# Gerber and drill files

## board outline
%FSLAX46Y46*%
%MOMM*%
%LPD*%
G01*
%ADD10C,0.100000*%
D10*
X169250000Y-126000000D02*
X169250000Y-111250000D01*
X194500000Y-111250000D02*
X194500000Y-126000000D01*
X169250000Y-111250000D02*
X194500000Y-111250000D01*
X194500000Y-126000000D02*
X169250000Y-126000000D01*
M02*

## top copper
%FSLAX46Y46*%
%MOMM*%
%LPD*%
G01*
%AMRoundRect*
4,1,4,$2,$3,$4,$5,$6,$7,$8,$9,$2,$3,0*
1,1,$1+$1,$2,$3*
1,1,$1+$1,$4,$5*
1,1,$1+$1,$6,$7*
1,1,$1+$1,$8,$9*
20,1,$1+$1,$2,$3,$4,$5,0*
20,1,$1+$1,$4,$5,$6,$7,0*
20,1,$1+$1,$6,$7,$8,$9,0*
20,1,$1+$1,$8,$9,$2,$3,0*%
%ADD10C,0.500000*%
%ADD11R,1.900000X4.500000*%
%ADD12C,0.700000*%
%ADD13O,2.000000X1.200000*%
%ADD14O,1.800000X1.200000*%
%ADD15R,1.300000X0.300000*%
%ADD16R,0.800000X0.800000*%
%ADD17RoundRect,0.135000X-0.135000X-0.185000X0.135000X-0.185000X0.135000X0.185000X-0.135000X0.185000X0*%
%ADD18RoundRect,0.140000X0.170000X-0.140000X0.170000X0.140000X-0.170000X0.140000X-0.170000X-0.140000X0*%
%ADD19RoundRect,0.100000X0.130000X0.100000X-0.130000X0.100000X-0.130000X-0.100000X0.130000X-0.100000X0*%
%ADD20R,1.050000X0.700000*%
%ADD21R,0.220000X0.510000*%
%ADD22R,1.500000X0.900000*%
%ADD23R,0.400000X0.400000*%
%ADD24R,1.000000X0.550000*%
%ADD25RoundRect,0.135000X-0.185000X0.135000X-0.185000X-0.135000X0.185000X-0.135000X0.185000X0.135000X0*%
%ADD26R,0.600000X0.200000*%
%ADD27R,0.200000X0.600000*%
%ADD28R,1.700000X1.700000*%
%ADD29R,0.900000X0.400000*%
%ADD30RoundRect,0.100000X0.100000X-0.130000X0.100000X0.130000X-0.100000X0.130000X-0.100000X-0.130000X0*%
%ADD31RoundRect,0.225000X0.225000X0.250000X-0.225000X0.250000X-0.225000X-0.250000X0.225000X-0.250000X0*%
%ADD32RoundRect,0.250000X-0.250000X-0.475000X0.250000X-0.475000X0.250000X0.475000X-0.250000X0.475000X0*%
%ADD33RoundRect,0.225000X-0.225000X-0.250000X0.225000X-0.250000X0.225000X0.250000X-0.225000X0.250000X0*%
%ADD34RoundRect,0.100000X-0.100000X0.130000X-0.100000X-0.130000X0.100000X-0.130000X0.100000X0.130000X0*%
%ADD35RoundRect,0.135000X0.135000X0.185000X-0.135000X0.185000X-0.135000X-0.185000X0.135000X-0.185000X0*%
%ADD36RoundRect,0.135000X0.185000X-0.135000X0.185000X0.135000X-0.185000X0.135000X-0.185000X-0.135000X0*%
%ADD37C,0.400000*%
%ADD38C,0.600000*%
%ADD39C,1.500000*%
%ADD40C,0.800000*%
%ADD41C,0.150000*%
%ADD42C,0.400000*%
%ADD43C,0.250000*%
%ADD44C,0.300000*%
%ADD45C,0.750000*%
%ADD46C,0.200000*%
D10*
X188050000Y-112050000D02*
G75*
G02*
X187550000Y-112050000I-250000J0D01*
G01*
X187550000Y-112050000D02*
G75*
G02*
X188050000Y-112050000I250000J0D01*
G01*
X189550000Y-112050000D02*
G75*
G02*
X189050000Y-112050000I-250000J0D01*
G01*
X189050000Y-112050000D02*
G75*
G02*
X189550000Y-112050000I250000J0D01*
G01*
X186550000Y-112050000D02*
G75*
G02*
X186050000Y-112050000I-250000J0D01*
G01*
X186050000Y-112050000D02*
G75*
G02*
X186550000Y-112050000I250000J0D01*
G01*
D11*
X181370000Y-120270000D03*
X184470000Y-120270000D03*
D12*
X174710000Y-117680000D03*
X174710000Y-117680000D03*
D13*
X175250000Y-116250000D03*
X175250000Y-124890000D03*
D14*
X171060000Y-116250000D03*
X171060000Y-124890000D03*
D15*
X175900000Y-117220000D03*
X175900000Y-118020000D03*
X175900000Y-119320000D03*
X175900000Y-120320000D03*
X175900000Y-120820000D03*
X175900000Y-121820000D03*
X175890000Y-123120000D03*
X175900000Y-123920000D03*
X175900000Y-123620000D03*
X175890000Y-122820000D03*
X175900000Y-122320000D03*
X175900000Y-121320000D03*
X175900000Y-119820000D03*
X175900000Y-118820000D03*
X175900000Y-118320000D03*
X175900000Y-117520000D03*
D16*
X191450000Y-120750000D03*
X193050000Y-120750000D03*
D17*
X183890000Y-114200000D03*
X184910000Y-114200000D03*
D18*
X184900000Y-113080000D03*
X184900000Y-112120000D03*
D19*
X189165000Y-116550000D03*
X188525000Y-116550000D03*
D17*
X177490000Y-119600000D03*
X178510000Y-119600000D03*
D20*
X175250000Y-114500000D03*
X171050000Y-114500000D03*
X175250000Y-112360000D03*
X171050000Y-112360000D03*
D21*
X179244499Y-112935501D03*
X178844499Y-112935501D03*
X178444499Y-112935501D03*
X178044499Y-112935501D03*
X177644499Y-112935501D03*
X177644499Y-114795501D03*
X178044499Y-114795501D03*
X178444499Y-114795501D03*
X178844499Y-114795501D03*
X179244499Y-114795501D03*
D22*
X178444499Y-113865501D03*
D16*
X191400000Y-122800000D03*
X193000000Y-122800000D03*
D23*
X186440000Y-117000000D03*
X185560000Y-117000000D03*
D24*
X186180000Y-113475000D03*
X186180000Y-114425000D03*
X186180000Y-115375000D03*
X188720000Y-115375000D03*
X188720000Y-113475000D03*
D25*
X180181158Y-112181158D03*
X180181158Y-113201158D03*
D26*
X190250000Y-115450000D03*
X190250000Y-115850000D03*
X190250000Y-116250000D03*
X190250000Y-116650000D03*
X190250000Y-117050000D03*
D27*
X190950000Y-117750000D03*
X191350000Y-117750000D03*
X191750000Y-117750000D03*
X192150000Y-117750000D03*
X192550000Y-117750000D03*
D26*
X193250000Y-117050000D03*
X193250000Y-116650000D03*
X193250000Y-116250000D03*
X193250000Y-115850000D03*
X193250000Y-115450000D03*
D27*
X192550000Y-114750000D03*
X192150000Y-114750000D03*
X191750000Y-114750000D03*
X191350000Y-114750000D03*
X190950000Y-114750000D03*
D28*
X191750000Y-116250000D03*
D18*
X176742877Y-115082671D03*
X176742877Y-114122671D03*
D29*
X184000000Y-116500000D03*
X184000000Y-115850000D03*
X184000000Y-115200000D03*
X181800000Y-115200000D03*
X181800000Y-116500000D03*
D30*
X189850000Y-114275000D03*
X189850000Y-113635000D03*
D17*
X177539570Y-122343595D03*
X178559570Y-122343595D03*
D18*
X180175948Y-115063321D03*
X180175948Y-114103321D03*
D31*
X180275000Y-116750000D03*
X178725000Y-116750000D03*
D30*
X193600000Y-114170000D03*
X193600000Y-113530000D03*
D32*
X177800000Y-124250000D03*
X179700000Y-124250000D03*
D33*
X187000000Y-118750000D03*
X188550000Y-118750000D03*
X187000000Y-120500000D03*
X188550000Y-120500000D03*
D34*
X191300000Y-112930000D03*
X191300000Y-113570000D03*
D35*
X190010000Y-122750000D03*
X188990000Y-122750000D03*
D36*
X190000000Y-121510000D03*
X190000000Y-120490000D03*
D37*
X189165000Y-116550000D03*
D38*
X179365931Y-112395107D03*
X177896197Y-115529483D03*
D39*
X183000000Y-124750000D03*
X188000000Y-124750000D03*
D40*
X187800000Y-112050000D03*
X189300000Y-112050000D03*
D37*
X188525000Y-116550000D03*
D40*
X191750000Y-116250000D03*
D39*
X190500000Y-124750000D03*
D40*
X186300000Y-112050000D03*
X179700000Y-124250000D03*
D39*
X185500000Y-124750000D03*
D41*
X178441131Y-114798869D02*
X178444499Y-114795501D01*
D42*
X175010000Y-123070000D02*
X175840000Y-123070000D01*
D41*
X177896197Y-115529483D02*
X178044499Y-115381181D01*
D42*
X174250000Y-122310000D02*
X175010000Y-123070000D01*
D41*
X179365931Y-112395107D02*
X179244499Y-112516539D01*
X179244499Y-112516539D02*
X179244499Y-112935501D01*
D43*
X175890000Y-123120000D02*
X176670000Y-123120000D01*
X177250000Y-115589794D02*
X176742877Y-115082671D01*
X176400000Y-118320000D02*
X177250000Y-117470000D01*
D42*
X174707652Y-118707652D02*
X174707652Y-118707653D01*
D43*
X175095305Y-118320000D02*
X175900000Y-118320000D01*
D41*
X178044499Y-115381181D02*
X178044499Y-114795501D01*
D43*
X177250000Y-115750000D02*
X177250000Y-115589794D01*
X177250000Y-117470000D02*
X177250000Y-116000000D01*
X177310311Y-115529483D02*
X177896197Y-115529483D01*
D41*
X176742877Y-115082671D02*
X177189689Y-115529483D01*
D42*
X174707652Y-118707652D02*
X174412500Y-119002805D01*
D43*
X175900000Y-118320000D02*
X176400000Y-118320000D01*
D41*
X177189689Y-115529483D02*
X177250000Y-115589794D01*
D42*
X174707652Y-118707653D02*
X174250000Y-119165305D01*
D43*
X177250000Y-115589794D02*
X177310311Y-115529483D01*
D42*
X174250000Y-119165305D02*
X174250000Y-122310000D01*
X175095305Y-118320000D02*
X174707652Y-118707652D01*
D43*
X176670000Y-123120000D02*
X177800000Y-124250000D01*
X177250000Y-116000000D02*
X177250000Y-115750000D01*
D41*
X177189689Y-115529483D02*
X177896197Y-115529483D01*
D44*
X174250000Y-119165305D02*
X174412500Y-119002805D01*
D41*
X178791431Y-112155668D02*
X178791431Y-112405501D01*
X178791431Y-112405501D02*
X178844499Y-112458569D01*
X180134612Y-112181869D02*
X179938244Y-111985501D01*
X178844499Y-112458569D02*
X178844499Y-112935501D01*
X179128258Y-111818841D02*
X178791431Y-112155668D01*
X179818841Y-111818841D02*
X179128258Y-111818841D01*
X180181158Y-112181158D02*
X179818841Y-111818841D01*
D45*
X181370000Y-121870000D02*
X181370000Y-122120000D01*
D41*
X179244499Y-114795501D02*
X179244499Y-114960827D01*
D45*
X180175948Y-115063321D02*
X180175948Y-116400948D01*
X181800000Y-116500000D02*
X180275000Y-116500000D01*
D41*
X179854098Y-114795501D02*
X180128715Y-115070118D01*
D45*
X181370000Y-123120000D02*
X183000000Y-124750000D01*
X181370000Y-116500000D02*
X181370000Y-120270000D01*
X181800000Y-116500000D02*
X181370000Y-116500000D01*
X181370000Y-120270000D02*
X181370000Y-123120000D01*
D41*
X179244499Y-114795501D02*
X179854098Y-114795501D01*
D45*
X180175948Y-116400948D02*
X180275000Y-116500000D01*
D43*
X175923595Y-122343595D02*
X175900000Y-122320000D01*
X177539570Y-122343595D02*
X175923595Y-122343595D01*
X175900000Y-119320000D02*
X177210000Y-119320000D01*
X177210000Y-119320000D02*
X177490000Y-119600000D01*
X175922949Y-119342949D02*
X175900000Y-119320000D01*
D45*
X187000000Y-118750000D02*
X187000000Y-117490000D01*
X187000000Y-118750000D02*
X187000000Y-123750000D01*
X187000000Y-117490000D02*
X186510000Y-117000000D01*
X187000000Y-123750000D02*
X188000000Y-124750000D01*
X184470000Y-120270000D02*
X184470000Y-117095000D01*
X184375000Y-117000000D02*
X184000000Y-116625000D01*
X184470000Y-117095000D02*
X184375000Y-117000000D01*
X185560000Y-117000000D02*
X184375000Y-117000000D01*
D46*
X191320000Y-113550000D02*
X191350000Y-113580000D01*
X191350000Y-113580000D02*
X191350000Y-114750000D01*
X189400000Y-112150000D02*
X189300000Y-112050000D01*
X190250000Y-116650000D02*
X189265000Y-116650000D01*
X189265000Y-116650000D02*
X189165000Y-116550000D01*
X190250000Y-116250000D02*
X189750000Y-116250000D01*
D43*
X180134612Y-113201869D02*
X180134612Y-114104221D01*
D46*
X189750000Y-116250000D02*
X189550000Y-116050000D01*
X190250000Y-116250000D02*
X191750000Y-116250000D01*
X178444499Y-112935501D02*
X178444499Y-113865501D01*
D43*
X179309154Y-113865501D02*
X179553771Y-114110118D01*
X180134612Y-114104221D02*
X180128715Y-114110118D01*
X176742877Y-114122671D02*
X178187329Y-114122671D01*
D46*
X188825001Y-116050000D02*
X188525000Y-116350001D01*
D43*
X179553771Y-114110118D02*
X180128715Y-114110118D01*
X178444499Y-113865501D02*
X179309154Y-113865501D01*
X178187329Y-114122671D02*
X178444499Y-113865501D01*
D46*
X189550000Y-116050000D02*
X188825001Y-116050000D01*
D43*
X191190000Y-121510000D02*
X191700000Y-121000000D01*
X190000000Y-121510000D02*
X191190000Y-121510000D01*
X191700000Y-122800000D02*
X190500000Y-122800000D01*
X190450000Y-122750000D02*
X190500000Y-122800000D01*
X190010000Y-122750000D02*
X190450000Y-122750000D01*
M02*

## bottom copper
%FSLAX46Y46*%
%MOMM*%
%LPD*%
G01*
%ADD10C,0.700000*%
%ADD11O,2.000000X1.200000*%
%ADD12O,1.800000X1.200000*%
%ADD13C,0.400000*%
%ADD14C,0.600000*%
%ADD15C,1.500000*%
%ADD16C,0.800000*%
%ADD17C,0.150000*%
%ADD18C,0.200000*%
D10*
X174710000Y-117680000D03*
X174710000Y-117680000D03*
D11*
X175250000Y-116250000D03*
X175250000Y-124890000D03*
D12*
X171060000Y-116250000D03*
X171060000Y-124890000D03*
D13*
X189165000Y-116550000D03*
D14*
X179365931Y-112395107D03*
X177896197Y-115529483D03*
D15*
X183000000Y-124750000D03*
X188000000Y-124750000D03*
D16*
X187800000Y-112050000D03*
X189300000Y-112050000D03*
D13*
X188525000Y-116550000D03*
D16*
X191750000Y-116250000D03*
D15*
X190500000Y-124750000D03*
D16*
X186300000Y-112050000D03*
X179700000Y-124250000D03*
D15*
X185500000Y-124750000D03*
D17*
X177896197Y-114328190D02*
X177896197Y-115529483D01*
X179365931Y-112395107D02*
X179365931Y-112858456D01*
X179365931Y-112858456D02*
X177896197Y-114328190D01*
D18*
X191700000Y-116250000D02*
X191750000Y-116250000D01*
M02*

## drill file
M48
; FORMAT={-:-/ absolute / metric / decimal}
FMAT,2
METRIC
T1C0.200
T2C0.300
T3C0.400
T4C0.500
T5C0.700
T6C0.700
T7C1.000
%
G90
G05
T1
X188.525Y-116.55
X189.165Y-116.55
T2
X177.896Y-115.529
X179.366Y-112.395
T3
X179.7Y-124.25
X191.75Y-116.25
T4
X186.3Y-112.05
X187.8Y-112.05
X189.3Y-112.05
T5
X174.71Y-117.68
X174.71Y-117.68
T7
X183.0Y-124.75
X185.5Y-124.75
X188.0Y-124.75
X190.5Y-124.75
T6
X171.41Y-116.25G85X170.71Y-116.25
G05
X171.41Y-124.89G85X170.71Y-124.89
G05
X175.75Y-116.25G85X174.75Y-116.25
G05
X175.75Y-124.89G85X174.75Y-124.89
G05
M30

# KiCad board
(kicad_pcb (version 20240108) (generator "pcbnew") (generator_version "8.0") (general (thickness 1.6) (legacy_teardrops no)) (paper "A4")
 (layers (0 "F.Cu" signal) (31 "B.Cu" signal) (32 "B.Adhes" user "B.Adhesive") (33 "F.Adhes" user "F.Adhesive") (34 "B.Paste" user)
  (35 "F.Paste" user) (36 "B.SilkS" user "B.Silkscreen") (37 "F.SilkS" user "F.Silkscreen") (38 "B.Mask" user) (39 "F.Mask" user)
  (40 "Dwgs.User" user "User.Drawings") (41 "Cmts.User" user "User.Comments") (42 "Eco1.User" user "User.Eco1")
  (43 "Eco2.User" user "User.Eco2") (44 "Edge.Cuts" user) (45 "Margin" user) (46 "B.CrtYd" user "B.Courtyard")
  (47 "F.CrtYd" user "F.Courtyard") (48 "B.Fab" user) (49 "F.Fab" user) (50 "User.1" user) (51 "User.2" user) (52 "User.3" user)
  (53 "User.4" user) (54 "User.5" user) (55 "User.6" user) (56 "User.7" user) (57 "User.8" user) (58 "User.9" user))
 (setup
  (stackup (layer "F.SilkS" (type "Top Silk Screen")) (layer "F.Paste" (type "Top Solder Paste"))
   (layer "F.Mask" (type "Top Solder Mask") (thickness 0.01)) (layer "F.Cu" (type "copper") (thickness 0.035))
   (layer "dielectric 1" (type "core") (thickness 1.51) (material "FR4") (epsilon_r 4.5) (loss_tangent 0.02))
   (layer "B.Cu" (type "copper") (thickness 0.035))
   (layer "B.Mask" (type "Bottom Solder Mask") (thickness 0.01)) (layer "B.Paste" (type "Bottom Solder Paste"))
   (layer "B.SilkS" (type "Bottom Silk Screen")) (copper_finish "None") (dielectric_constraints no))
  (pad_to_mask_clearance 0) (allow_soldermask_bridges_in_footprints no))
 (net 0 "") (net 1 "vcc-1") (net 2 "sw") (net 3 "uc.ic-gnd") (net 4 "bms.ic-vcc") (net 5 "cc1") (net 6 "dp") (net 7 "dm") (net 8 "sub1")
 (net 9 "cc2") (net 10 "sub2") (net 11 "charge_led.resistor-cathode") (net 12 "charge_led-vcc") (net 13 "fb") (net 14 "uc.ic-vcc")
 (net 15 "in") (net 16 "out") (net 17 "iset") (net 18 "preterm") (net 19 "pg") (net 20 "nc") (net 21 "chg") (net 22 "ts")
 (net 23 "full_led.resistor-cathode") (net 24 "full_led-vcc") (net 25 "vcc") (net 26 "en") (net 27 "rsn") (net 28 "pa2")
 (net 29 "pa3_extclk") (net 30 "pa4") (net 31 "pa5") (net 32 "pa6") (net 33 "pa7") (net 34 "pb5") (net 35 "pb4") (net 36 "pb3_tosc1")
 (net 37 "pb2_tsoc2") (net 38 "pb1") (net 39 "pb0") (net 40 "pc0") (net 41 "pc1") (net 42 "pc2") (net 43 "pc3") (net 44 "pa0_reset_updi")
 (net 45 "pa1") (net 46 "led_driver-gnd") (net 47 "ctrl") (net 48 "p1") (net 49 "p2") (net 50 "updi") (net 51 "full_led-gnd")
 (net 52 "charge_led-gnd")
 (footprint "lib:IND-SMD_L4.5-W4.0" (layer "F.Cu") (at 182.92 120.27)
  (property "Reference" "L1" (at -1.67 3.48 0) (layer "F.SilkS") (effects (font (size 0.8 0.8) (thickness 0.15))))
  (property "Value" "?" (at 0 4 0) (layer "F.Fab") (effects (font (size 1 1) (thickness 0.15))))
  (pad "1" smd rect (at -1.55 0) (size 1.9 4.5) (layers "F.Cu" "F.Paste" "F.Mask") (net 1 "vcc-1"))
  (pad "2" smd rect (at 1.55 0) (size 1.9 4.5) (layers "F.Cu" "F.Paste" "F.Mask") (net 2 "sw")))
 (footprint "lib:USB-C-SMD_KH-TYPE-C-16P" (layer "F.Cu") (at 173.48 120.57 -90)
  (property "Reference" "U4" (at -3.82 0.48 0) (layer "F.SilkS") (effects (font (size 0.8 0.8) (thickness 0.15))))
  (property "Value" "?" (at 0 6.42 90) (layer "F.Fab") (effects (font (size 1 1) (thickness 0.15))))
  (pad "" thru_hole circle (at -2.89 -1.23 270) (size 0.7 0.7) (drill 0.7) (layers "*.Cu" "*.Mask") (remove_unused_layers no))
  (pad "" thru_hole circle (at -2.89 -1.23 270) (size 0.7 0.7) (drill 0.7) (layers "*.Cu" "*.Mask") (remove_unused_layers no))
  (pad "1" thru_hole oval (at -4.32 -1.77 270) (size 1.2 2) (drill oval 0.700024 1.699997) (layers "*.Cu" "*.Mask")
   (remove_unused_layers no) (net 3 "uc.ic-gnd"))
  (pad "2" thru_hole oval (at 4.32 -1.77 270) (size 1.2 2) (drill oval 0.700024 1.699997) (layers "*.Cu" "*.Mask") (remove_unused_layers no)
   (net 3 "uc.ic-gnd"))
  (pad "3" thru_hole oval (at -4.32 2.42 270) (size 1.2 1.8) (drill oval 0.700024 1.399997) (layers "*.Cu" "*.Mask")
   (remove_unused_layers no) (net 3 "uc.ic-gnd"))
  (pad "4" thru_hole oval (at 4.32 2.42 270) (size 1.2 1.8) (drill oval 0.700024 1.399997) (layers "*.Cu" "*.Mask")
   (remove_unused_layers no) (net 3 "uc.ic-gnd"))
  (pad "A1" smd rect (at -3.35 -2.42 270) (size 0.3 1.3) (layers "F.Cu" "F.Paste" "F.Mask") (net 3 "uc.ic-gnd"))
  (pad "A4" smd rect (at -2.55 -2.42 270) (size 0.3 1.3) (layers "F.Cu" "F.Paste" "F.Mask") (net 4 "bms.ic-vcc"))
  (pad "A5" smd rect (at -1.25 -2.42 270) (size 0.3 1.3) (layers "F.Cu" "F.Paste" "F.Mask") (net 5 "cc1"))
  (pad "A6" smd rect (at -0.25 -2.42 270) (size 0.3 1.3) (layers "F.Cu" "F.Paste" "F.Mask") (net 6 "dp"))
  (pad "A7" smd rect (at 0.25 -2.42 270) (size 0.3 1.3) (layers "F.Cu" "F.Paste" "F.Mask") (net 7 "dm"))
  (pad "A8" smd rect (at 1.25 -2.42 270) (size 0.3 1.3) (layers "F.Cu" "F.Paste" "F.Mask") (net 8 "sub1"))
  (pad "A9" smd rect (at 2.55 -2.41 270) (size 0.3 1.3) (layers "F.Cu" "F.Paste" "F.Mask") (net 4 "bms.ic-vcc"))
  (pad "A12" smd rect (at 3.35 -2.42 270) (size 0.3 1.3) (layers "F.Cu" "F.Paste" "F.Mask") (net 3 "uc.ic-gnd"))
  (pad "B1" smd rect (at 3.05 -2.42 270) (size 0.3 1.3) (layers "F.Cu" "F.Paste" "F.Mask") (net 3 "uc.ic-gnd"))
  (pad "B4" smd rect (at 2.25 -2.41 270) (size 0.3 1.3) (layers "F.Cu" "F.Paste" "F.Mask") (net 4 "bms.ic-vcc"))
  (pad "B5" smd rect (at 1.75 -2.42 270) (size 0.3 1.3) (layers "F.Cu" "F.Paste" "F.Mask") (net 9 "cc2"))
  (pad "B6" smd rect (at 0.75 -2.42 270) (size 0.3 1.3) (layers "F.Cu" "F.Paste" "F.Mask") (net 6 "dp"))
  (pad "B7" smd rect (at -0.75 -2.42 270) (size 0.3 1.3) (layers "F.Cu" "F.Paste" "F.Mask") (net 7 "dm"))
  (pad "B8" smd rect (at -1.75 -2.42 270) (size 0.3 1.3) (layers "F.Cu" "F.Paste" "F.Mask") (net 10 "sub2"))
  (pad "B9" smd rect (at -2.25 -2.42 270) (size 0.3 1.3) (layers "F.Cu" "F.Paste" "F.Mask") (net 4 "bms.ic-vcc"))
  (pad "B12" smd rect (at -3.05 -2.42 270) (size 0.3 1.3) (layers "F.Cu" "F.Paste" "F.Mask") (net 3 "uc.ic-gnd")))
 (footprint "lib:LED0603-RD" (layer "F.Cu") (at 192.25 120.75)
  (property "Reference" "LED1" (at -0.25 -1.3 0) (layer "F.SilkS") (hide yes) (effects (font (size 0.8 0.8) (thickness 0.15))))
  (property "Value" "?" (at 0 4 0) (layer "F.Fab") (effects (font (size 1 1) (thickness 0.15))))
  (pad "1" smd rect (at -0.8 0 90) (size 0.8 0.8) (layers "F.Cu" "F.Paste" "F.Mask") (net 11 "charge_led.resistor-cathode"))
  (pad "2" smd rect (at 0.8 0 90) (size 0.8 0.8) (layers "F.Cu" "F.Paste" "F.Mask") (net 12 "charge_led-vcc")))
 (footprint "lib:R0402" (layer "F.Cu") (at 184.4 114.2)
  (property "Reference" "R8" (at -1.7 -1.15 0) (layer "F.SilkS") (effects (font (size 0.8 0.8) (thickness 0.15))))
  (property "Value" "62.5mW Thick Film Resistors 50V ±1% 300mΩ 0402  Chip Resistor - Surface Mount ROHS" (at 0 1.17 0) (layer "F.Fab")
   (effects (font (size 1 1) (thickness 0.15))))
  (pad "1" smd roundrect (at -0.51 0) (size 0.54 0.64) (layers "F.Cu" "F.Paste" "F.Mask") (roundrect_rratio 0.25) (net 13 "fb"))
  (pad "2" smd roundrect (at 0.51 0) (size 0.54 0.64) (layers "F.Cu" "F.Paste" "F.Mask") (roundrect_rratio 0.25) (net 3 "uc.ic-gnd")))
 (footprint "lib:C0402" (layer "F.Cu") (at 184.9 112.6 90)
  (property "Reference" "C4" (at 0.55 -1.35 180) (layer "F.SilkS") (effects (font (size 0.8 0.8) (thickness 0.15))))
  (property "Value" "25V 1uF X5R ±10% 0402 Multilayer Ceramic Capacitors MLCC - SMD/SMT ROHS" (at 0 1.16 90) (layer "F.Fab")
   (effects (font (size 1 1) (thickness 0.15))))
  (pad "1" smd roundrect (at -0.48 0 90) (size 0.56 0.62) (layers "F.Cu" "F.Paste" "F.Mask") (roundrect_rratio 0.25) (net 1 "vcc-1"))
  (pad "2" smd roundrect (at 0.48 0 90) (size 0.56 0.62) (layers "F.Cu" "F.Paste" "F.Mask") (roundrect_rratio 0.25) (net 3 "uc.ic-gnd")))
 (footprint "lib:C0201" (layer "F.Cu") (at 188.845 116.55 180)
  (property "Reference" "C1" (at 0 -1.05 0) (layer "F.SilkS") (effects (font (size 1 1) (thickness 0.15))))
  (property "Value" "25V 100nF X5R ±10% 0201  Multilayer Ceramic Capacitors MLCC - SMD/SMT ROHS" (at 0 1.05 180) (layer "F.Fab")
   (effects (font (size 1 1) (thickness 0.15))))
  (pad "" smd roundrect (at -0.345 0 180) (size 0.318 0.36) (layers "F.Paste") (roundrect_rratio 0.25))
  (pad "" smd roundrect (at -0.345 0 180) (size 0.318 0.36) (layers "F.Paste") (roundrect_rratio 0.25))
  (pad "1" smd roundrect (at -0.32 0 180) (size 0.46 0.4) (layers "F.Cu" "F.Mask") (roundrect_rratio 0.25) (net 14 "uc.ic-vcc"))
  (pad "2" smd roundrect (at 0.32 0 180) (size 0.46 0.4) (layers "F.Cu" "F.Mask") (roundrect_rratio 0.25) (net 3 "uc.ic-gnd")))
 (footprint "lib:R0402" (layer "F.Cu") (at 178 119.6)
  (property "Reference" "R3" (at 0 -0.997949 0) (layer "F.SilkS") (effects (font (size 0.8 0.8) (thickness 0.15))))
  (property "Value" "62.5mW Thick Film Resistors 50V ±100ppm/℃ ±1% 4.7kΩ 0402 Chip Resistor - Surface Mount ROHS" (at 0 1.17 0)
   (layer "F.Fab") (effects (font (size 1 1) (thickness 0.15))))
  (pad "1" smd roundrect (at -0.51 0) (size 0.54 0.64) (layers "F.Cu" "F.Paste" "F.Mask") (roundrect_rratio 0.25) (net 5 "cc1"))
  (pad "2" smd roundrect (at 0.51 0) (size 0.54 0.64) (layers "F.Cu" "F.Paste" "F.Mask") (roundrect_rratio 0.25) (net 3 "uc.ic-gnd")))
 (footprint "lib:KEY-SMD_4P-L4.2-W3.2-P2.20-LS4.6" (layer "F.Cu") (at 173.15 113.43 180)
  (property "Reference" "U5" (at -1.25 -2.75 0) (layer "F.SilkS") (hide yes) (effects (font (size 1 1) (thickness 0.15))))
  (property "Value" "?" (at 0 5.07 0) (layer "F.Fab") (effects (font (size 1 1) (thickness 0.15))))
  (pad "1" smd rect (at -2.1 -1.07 180) (size 1.05 0.7) (layers "F.Cu" "F.Paste" "F.Mask") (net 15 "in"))
  (pad "2" smd rect (at 2.1 -1.07 180) (size 1.05 0.7) (layers "F.Cu" "F.Paste" "F.Mask") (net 15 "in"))
  (pad "3" smd rect (at -2.1 1.07 180) (size 1.05 0.7) (layers "F.Cu" "F.Paste" "F.Mask") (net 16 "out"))
  (pad "4" smd rect (at 2.1 1.07 180) (size 1.05 0.7) (layers "F.Cu" "F.Paste" "F.Mask") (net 16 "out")))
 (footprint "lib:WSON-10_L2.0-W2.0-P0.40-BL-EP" (layer "F.Cu") (at 178.444499 113.865501 180)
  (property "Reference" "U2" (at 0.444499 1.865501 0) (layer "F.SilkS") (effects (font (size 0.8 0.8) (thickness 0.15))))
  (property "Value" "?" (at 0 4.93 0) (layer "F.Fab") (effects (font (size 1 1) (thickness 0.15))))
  (pad "1" smd rect (at -0.8 0.93 180) (size 0.22 0.51) (layers "F.Cu" "F.Paste" "F.Mask") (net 4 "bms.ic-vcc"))
  (pad "2" smd rect (at -0.4 0.93 180) (size 0.22 0.51) (layers "F.Cu" "F.Paste" "F.Mask") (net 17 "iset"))
  (pad "3" smd rect (at 0 0.93 180) (size 0.22 0.51) (layers "F.Cu" "F.Paste" "F.Mask") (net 3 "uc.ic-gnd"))
  (pad "4" smd rect (at 0.4 0.93 180) (size 0.22 0.51) (layers "F.Cu" "F.Paste" "F.Mask") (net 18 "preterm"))
  (pad "5" smd rect (at 0.8 0.93 180) (size 0.22 0.51) (layers "F.Cu" "F.Paste" "F.Mask") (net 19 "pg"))
  (pad "6" smd rect (at 0.8 -0.93 180) (size 0.22 0.51) (layers "F.Cu" "F.Paste" "F.Mask") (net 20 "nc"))
  (pad "7" smd rect (at 0.4 -0.93 180) (size 0.22 0.51) (layers "F.Cu" "F.Paste" "F.Mask") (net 4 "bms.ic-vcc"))
  (pad "8" smd rect (at 0 -0.93 180) (size 0.22 0.51) (layers "F.Cu" "F.Paste" "F.Mask") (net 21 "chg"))
  (pad "9" smd rect (at -0.4 -0.93 180) (size 0.22 0.51) (layers "F.Cu" "F.Paste" "F.Mask") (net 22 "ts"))
  (pad "10" smd rect (at -0.8 -0.93 180) (size 0.22 0.51) (layers "F.Cu" "F.Paste" "F.Mask") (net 1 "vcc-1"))
  (pad "11" smd rect (at 0 0 180) (size 1.5 0.9) (layers "F.Cu" "F.Paste" "F.Mask") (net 3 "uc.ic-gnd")))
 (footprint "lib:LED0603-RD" (layer "F.Cu") (at 192.2 122.8)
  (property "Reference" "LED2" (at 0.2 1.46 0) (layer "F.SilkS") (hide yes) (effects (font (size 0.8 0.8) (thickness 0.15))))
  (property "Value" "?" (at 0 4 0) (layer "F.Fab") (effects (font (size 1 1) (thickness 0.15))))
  (pad "1" smd rect (at -0.8 0 90) (size 0.8 0.8) (layers "F.Cu" "F.Paste" "F.Mask") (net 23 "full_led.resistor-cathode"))
  (pad "2" smd rect (at 0.8 0 90) (size 0.8 0.8) (layers "F.Cu" "F.Paste" "F.Mask") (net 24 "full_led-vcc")))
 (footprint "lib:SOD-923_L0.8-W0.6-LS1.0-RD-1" (layer "F.Cu") (at 186 117 180)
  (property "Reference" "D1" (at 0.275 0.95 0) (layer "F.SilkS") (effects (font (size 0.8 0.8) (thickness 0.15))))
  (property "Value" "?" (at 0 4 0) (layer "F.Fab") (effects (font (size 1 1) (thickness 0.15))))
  (pad "1" smd rect (at -0.44 0) (size 0.4 0.4) (layers "F.Cu" "F.Paste" "F.Mask") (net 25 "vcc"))
  (pad "2" smd rect (at 0.44 0) (size 0.4 0.4) (layers "F.Cu" "F.Paste" "F.Mask") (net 2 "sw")))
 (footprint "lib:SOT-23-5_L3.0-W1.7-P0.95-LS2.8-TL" (layer "F.Cu") (at 187.45 114.425)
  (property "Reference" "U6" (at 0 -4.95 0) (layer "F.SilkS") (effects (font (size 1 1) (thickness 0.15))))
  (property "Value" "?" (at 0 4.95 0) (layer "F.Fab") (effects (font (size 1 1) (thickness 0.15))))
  (pad "1" smd rect (at -1.27 -0.95 270) (size 0.55 1) (layers "F.Cu" "F.Paste" "F.Mask") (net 1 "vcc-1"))
  (pad "2" smd rect (at -1.27 0 270) (size 0.55 1) (layers "F.Cu" "F.Paste" "F.Mask") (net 3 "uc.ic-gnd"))
  (pad "3" smd rect (at -1.27 0.95 270) (size 0.55 1) (layers "F.Cu" "F.Paste" "F.Mask") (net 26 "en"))
  (pad "4" smd rect (at 1.27 0.95 270) (size 0.55 1) (layers "F.Cu" "F.Paste" "F.Mask") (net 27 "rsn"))
  (pad "5" smd rect (at 1.27 -0.95 270) (size 0.55 1) (layers "F.Cu" "F.Paste" "F.Mask") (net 14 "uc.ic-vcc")))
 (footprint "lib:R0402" (layer "F.Cu") (at 180.181158 112.691158 -90)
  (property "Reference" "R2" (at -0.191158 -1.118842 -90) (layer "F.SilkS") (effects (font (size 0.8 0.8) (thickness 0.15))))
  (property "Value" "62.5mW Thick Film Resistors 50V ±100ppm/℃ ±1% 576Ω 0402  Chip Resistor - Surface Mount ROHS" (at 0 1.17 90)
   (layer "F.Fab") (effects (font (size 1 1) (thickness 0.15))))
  (pad "1" smd roundrect (at -0.51 0 270) (size 0.54 0.64) (layers "F.Cu" "F.Paste" "F.Mask") (roundrect_rratio 0.25) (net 17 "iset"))
  (pad "2" smd roundrect (at 0.51 0 270) (size 0.54 0.64) (layers "F.Cu" "F.Paste" "F.Mask") (roundrect_rratio 0.25) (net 3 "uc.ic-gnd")))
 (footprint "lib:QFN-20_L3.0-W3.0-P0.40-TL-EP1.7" (layer "F.Cu") (at 191.75 116.25)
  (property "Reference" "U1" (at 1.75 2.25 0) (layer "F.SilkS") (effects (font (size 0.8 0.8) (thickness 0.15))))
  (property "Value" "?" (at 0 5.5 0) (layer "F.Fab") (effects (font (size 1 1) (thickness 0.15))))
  (pad "1" smd rect (at -1.5 -0.8) (size 0.6 0.2) (layers "F.Cu" "F.Paste" "F.Mask") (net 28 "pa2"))
  (pad "2" smd rect (at -1.5 -0.4) (size 0.6 0.2) (layers "F.Cu" "F.Paste" "F.Mask") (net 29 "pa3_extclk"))
  (pad "3" smd rect (at -1.5 0) (size 0.6 0.2) (layers "F.Cu" "F.Paste" "F.Mask") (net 3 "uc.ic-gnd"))
  (pad "4" smd rect (at -1.5 0.4) (size 0.6 0.2) (layers "F.Cu" "F.Paste" "F.Mask") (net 14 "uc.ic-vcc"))
  (pad "5" smd rect (at -1.5 0.8) (size 0.6 0.2) (layers "F.Cu" "F.Paste" "F.Mask") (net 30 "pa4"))
  (pad "6" smd rect (at -0.8 1.5) (size 0.2 0.6) (layers "F.Cu" "F.Paste" "F.Mask") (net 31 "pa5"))
  (pad "7" smd rect (at -0.4 1.5) (size 0.2 0.6) (layers "F.Cu" "F.Paste" "F.Mask") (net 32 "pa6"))
  (pad "8" smd rect (at 0 1.5) (size 0.2 0.6) (layers "F.Cu" "F.Paste" "F.Mask") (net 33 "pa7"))
  (pad "9" smd rect (at 0.4 1.5) (size 0.2 0.6) (layers "F.Cu" "F.Paste" "F.Mask") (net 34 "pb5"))
  (pad "10" smd rect (at 0.8 1.5) (size 0.2 0.6) (layers "F.Cu" "F.Paste" "F.Mask") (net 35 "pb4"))
  (pad "11" smd rect (at 1.5 0.8) (size 0.6 0.2) (layers "F.Cu" "F.Paste" "F.Mask") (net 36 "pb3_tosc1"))
  (pad "12" smd rect (at 1.5 0.4) (size 0.6 0.2) (layers "F.Cu" "F.Paste" "F.Mask") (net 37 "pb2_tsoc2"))
  (pad "13" smd rect (at 1.5 0) (size 0.6 0.2) (layers "F.Cu" "F.Paste" "F.Mask") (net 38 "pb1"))
  (pad "14" smd rect (at 1.5 -0.4) (size 0.6 0.2) (layers "F.Cu" "F.Paste" "F.Mask") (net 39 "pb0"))
  (pad "15" smd rect (at 1.5 -0.8) (size 0.6 0.2) (layers "F.Cu" "F.Paste" "F.Mask") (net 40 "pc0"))
  (pad "16" smd rect (at 0.8 -1.5) (size 0.2 0.6) (layers "F.Cu" "F.Paste" "F.Mask") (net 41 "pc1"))
  (pad "17" smd rect (at 0.4 -1.5) (size 0.2 0.6) (layers "F.Cu" "F.Paste" "F.Mask") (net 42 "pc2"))
  (pad "18" smd rect (at 0 -1.5) (size 0.2 0.6) (layers "F.Cu" "F.Paste" "F.Mask") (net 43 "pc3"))
  (pad "19" smd rect (at -0.4 -1.5) (size 0.2 0.6) (layers "F.Cu" "F.Paste" "F.Mask") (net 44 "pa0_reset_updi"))
  (pad "20" smd rect (at -0.8 -1.5) (size 0.2 0.6) (layers "F.Cu" "F.Paste" "F.Mask") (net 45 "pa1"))
  (pad "21" smd rect (at 0 0 180) (size 1.7 1.7) (layers "F.Cu" "F.Paste" "F.Mask") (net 3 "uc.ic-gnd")))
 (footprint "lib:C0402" (layer "F.Cu") (at 176.742877 114.602671 90)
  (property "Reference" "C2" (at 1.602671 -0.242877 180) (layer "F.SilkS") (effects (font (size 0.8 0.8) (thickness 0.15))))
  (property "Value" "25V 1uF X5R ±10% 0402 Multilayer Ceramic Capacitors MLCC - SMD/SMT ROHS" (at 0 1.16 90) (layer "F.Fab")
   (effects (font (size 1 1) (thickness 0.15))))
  (pad "1" smd roundrect (at -0.48 0 90) (size 0.56 0.62) (layers "F.Cu" "F.Paste" "F.Mask") (roundrect_rratio 0.25) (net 4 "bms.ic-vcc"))
  (pad "2" smd roundrect (at 0.48 0 90) (size 0.56 0.62) (layers "F.Cu" "F.Paste" "F.Mask") (roundrect_rratio 0.25) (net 3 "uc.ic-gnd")))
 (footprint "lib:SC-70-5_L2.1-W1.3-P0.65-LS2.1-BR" (layer "F.Cu") (at 182.9 115.85)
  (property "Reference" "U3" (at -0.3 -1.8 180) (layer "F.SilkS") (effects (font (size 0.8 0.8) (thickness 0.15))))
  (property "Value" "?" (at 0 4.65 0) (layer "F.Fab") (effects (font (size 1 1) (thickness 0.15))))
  (pad "1" smd rect (at 1.1 0.65 90) (size 0.4 0.9) (layers "F.Cu" "F.Paste" "F.Mask") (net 2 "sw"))
  (pad "2" smd rect (at 1.1 0 90) (size 0.4 0.9) (layers "F.Cu" "F.Paste" "F.Mask") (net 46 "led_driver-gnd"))
  (pad "3" smd rect (at 1.1 -0.65 90) (size 0.4 0.9) (layers "F.Cu" "F.Paste" "F.Mask") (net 13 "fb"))
  (pad "4" smd rect (at -1.1 -0.65 90) (size 0.4 0.9) (layers "F.Cu" "F.Paste" "F.Mask") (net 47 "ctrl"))
  (pad "5" smd rect (at -1.1 0.65 90) (size 0.4 0.9) (layers "F.Cu" "F.Paste" "F.Mask") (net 1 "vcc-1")))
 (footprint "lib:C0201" (layer "F.Cu") (at 189.85 113.955 90)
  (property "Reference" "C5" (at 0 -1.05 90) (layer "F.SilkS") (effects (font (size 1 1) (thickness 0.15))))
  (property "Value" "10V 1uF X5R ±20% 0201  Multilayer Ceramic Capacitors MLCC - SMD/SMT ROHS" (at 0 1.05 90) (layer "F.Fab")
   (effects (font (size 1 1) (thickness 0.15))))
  (pad "" smd roundrect (at -0.345 0 90) (size 0.318 0.36) (layers "F.Paste") (roundrect_rratio 0.25))
  (pad "" smd roundrect (at 0.345 0 90) (size 0.318 0.36) (layers "F.Paste") (roundrect_rratio 0.25))
  (pad "1" smd roundrect (at -0.32 0 90) (size 0.46 0.4) (layers "F.Cu" "F.Mask") (roundrect_rratio 0.25) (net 14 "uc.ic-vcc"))
  (pad "2" smd roundrect (at 0.32 0 90) (size 0.46 0.4) (layers "F.Cu" "F.Mask") (roundrect_rratio 0.25) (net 3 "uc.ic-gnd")))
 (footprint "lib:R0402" (layer "F.Cu") (at 178.04957 122.343595)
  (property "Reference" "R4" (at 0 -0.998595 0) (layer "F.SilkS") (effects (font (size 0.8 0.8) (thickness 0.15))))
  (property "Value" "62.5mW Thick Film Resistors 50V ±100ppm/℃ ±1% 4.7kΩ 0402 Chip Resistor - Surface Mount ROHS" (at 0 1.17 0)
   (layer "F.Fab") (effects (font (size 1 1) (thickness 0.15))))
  (pad "1" smd roundrect (at -0.51 0) (size 0.54 0.64) (layers "F.Cu" "F.Paste" "F.Mask") (roundrect_rratio 0.25) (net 9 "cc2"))
  (pad "2" smd roundrect (at 0.51 0) (size 0.54 0.64) (layers "F.Cu" "F.Paste" "F.Mask") (roundrect_rratio 0.25) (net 3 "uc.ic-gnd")))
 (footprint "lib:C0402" (layer "F.Cu") (at 180.175948 114.583321 90)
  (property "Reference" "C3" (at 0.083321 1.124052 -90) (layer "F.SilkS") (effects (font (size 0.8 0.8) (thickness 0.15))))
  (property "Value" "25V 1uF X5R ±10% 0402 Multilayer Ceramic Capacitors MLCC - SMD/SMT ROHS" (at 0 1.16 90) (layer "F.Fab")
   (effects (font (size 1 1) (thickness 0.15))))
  (pad "1" smd roundrect (at -0.48 0 90) (size 0.56 0.62) (layers "F.Cu" "F.Paste" "F.Mask") (roundrect_rratio 0.25) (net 1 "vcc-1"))
  (pad "2" smd roundrect (at 0.48 0 90) (size 0.56 0.62) (layers "F.Cu" "F.Paste" "F.Mask") (roundrect_rratio 0.25) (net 3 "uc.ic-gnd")))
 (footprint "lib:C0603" (layer "F.Cu") (at 179.5 116.75 180)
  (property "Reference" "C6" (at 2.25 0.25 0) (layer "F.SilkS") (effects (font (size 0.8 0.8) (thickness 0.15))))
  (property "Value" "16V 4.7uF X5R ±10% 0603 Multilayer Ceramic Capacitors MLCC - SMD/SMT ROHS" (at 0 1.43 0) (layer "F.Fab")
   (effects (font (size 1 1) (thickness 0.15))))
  (pad "1" smd roundrect (at -0.775 0 180) (size 0.9 0.95) (layers "F.Cu" "F.Paste" "F.Mask") (roundrect_rratio 0.25) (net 1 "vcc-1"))
  (pad "2" smd roundrect (at 0.775 0 180) (size 0.9 0.95) (layers "F.Cu" "F.Paste" "F.Mask") (roundrect_rratio 0.25) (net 3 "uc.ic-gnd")))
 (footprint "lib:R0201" (layer "F.Cu") (at 193.6 113.85 90)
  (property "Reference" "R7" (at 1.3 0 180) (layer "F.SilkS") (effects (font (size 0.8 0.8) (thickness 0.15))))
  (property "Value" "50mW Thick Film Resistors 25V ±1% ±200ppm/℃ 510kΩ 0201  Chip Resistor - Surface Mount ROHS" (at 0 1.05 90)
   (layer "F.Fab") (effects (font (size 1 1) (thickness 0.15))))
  (pad "" smd roundrect (at -0.345 0 90) (size 0.318 0.36) (layers "F.Paste") (roundrect_rratio 0.25))
  (pad "" smd roundrect (at 0.345 0 90) (size 0.318 0.36) (layers "F.Paste") (roundrect_rratio 0.25))
  (pad "1" smd roundrect (at -0.32 0 90) (size 0.46 0.4) (layers "F.Cu" "F.Mask") (roundrect_rratio 0.25) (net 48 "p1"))
  (pad "2" smd roundrect (at 0.32 0 90) (size 0.46 0.4) (layers "F.Cu" "F.Mask") (roundrect_rratio 0.25) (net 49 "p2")))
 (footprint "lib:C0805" (layer "F.Cu") (at 178.75 124.25)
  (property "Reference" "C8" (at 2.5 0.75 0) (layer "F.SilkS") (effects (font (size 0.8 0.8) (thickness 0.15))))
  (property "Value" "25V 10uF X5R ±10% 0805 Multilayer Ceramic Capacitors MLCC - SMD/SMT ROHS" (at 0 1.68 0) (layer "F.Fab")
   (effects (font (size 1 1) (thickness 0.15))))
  (pad "1" smd roundrect (at -0.95 0) (size 1 1.45) (layers "F.Cu" "F.Paste" "F.Mask") (roundrect_rratio 0.25) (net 4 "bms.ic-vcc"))
  (pad "2" smd roundrect (at 0.95 0) (size 1 1.45) (layers "F.Cu" "F.Paste" "F.Mask") (roundrect_rratio 0.25) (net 3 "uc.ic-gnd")))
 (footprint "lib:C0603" (layer "F.Cu") (at 187.775 118.75)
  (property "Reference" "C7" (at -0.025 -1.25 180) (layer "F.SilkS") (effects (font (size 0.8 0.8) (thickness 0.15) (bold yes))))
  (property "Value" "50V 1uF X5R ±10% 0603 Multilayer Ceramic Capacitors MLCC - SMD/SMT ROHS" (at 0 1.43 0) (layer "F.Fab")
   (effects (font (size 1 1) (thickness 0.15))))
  (pad "1" smd roundrect (at -0.775 0) (size 0.9 0.95) (layers "F.Cu" "F.Paste" "F.Mask") (roundrect_rratio 0.25) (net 25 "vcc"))
  (pad "2" smd roundrect (at 0.775 0) (size 0.9 0.95) (layers "F.Cu" "F.Paste" "F.Mask") (roundrect_rratio 0.25) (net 3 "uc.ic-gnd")))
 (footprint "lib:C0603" (layer "F.Cu") (at 187.775 120.5)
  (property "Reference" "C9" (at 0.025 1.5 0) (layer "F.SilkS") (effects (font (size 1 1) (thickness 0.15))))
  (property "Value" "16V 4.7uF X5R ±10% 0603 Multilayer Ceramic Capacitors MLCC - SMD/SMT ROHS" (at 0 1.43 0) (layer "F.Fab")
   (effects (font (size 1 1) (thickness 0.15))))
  (pad "1" smd roundrect (at -0.775 0) (size 0.9 0.95) (layers "F.Cu" "F.Paste" "F.Mask") (roundrect_rratio 0.25) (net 25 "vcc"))
  (pad "2" smd roundrect (at 0.775 0) (size 0.9 0.95) (layers "F.Cu" "F.Paste" "F.Mask") (roundrect_rratio 0.25) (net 3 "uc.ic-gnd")))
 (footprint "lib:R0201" (layer "F.Cu") (at 191.3 113.25 -90)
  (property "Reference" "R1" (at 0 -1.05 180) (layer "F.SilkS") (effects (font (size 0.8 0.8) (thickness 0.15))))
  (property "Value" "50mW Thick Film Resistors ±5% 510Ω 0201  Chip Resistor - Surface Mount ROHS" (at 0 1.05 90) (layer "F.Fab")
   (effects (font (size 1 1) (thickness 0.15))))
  (pad "" smd roundrect (at -0.345 0 270) (size 0.318 0.36) (layers "F.Paste") (roundrect_rratio 0.25))
  (pad "" smd roundrect (at -0.345 0 270) (size 0.318 0.36) (layers "F.Paste") (roundrect_rratio 0.25))
  (pad "1" smd roundrect (at -0.32 0 270) (size 0.46 0.4) (layers "F.Cu" "F.Mask") (roundrect_rratio 0.25) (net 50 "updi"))
  (pad "2" smd roundrect (at 0.32 0 270) (size 0.46 0.4) (layers "F.Cu" "F.Mask") (roundrect_rratio 0.25) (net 44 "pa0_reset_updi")))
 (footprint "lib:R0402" (layer "F.Cu") (at 189.5 122.75 180)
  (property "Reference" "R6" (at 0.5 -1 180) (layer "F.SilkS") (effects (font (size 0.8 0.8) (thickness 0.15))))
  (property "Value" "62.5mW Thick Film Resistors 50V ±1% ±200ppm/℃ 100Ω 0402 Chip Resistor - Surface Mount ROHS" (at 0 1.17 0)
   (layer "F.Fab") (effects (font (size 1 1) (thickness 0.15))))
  (pad "1" smd roundrect (at -0.51 0 180) (size 0.54 0.64) (layers "F.Cu" "F.Paste" "F.Mask") (roundrect_rratio 0.25)
   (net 23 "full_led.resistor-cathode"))
  (pad "2" smd roundrect (at 0.51 0 180) (size 0.54 0.64) (layers "F.Cu" "F.Paste" "F.Mask") (roundrect_rratio 0.25) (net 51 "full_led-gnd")))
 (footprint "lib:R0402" (layer "F.Cu") (at 190 121 90)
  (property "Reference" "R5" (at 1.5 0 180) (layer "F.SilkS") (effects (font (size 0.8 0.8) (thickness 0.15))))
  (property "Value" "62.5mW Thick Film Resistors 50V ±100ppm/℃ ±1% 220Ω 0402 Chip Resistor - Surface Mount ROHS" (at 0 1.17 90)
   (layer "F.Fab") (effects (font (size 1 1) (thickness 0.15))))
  (pad "1" smd roundrect (at -0.51 0 90) (size 0.54 0.64) (layers "F.Cu" "F.Paste" "F.Mask") (roundrect_rratio 0.25)
   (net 11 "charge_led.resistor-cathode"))
  (pad "2" smd roundrect (at 0.51 0 90) (size 0.54 0.64) (layers "F.Cu" "F.Paste" "F.Mask") (roundrect_rratio 0.25)
   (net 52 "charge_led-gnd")))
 (gr_circle (center 187.8 112.05) (end 188.2 112.05) (stroke (width 0.2) (type solid)) (fill solid) (layer "F.Cu") (net 25))
 (gr_circle (center 189.3 112.05) (end 189.7 112.05) (stroke (width 0.2) (type solid)) (fill solid) (layer "F.Cu") (net 50))
 (gr_circle (center 186.3 112.05) (end 186.7 112.05) (stroke (width 0.2) (type solid)) (fill solid) (layer "F.Cu") (net 3))
 (gr_line (start 169.25 126) (end 169.25 111.25) (stroke (width 0.1) (type default)) (layer "Edge.Cuts"))
 (gr_line (start 194.5 111.25) (end 194.5 126) (stroke (width 0.1) (type default)) (layer "Edge.Cuts"))
 (gr_line (start 169.25 111.25) (end 194.5 111.25) (stroke (width 0.1) (type default)) (layer "Edge.Cuts"))
 (gr_line (start 194.5 126) (end 169.25 126) (stroke (width 0.1) (type default)) (layer "Edge.Cuts"))
 (via (at 189.165 116.55) (size 0.4) (drill 0.2) (layers "F.Cu" "B.Cu") (free yes) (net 20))
 (segment (start 178.441131 114.798869) (end 178.444499 114.795501) (width 0.15) (layer "F.Cu") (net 21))
 (segment (start 175.01 123.07) (end 175.84 123.07) (width 0.4) (layer "F.Cu") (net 4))
 (segment (start 177.896197 115.529483) (end 178.044499 115.381181) (width 0.15) (layer "F.Cu") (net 4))
 (segment (start 174.25 122.31) (end 175.01 123.07) (width 0.4) (layer "F.Cu") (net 4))
 (segment (start 179.365931 112.395107) (end 179.244499 112.516539) (width 0.15) (layer "F.Cu") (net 4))
 (segment (start 179.244499 112.516539) (end 179.244499 112.935501) (width 0.15) (layer "F.Cu") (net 4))
 (segment (start 175.89 123.12) (end 176.67 123.12) (width 0.25) (layer "F.Cu") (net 4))
 (segment (start 177.25 115.589794) (end 176.742877 115.082671) (width 0.25) (layer "F.Cu") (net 4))
 (segment (start 176.4 118.32) (end 177.25 117.47) (width 0.25) (layer "F.Cu") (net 4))
 (segment (start 174.707652 118.707652) (end 174.707652 118.707653) (width 0.4) (layer "F.Cu") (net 4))
 (segment (start 175.095305 118.32) (end 175.9 118.32) (width 0.25) (layer "F.Cu") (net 4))
 (segment (start 178.044499 115.381181) (end 178.044499 114.795501) (width 0.15) (layer "F.Cu") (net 4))
 (segment (start 177.25 115.75) (end 177.25 115.589794) (width 0.25) (layer "F.Cu") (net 4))
 (segment (start 177.25 117.47) (end 177.25 116) (width 0.25) (layer "F.Cu") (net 4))
 (segment (start 177.310311 115.529483) (end 177.896197 115.529483) (width 0.25) (layer "F.Cu") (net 4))
 (segment (start 176.742877 115.082671) (end 177.189689 115.529483) (width 0.15) (layer "F.Cu") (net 4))
 (segment (start 174.707652 118.707652) (end 174.4125 119.002805) (width 0.4) (layer "F.Cu") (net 4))
 (segment (start 175.9 118.32) (end 176.4 118.32) (width 0.25) (layer "F.Cu") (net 4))
 (segment (start 177.189689 115.529483) (end 177.25 115.589794) (width 0.15) (layer "F.Cu") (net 4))
 (segment (start 174.707652 118.707653) (end 174.25 119.165305) (width 0.4) (layer "F.Cu") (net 4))
 (segment (start 177.25 115.589794) (end 177.310311 115.529483) (width 0.25) (layer "F.Cu") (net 4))
 (segment (start 174.25 119.165305) (end 174.25 122.31) (width 0.4) (layer "F.Cu") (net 4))
 (segment (start 175.095305 118.32) (end 174.707652 118.707652) (width 0.4) (layer "F.Cu") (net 4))
 (segment (start 176.67 123.12) (end 177.8 124.25) (width 0.25) (layer "F.Cu") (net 4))
 (segment (start 177.25 116) (end 177.25 115.75) (width 0.25) (layer "F.Cu") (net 4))
 (segment (start 177.189689 115.529483) (end 177.896197 115.529483) (width 0.15) (layer "F.Cu") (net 4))
 (segment (start 174.25 119.165305) (end 174.4125 119.002805) (width 0.3) (layer "F.Cu") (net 4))
 (via (at 179.365931 112.395107) (size 0.6) (drill 0.3) (layers "F.Cu" "B.Cu") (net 4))
 (via (at 177.896197 115.529483) (size 0.6) (drill 0.3) (layers "F.Cu" "B.Cu") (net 4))
 (segment (start 177.896197 114.32819) (end 177.896197 115.529483) (width 0.15) (layer "B.Cu") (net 4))
 (segment (start 179.365931 112.395107) (end 179.365931 112.858456) (width 0.15) (layer "B.Cu") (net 4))
 (segment (start 179.365931 112.858456) (end 177.896197 114.32819) (width 0.15) (layer "B.Cu") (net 4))
 (segment (start 178.791431 112.155668) (end 178.791431 112.405501) (width 0.15) (layer "F.Cu") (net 17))
 (segment (start 178.791431 112.405501) (end 178.844499 112.458569) (width 0.15) (layer "F.Cu") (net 17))
 (segment (start 180.134612 112.181869) (end 179.938244 111.985501) (width 0.15) (layer "F.Cu") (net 17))
 (segment (start 178.844499 112.458569) (end 178.844499 112.935501) (width 0.15) (layer "F.Cu") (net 17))
 (segment (start 179.128258 111.818841) (end 178.791431 112.155668) (width 0.15) (layer "F.Cu") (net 17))
 (segment (start 179.818841 111.818841) (end 179.128258 111.818841) (width 0.15) (layer "F.Cu") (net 17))
 (segment (start 180.181158 112.181158) (end 179.818841 111.818841) (width 0.15) (layer "F.Cu") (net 17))
 (segment (start 181.37 121.87) (end 181.37 122.12) (width 0.75) (layer "F.Cu") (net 1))
 (segment (start 179.244499 114.795501) (end 179.244499 114.960827) (width 0.15) (layer "F.Cu") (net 1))
 (segment (start 180.175948 115.063321) (end 180.175948 116.400948) (width 0.75) (layer "F.Cu") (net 1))
 (segment (start 181.8 116.5) (end 180.275 116.5) (width 0.75) (layer "F.Cu") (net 1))
 (segment (start 179.854098 114.795501) (end 180.128715 115.070118) (width 0.15) (layer "F.Cu") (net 1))
 (segment (start 181.37 123.12) (end 183 124.75) (width 0.75) (layer "F.Cu") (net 1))
 (segment (start 181.37 116.5) (end 181.37 120.27) (width 0.75) (layer "F.Cu") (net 1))
 (segment (start 181.8 116.5) (end 181.37 116.5) (width 0.75) (layer "F.Cu") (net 1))
 (segment (start 181.37 120.27) (end 181.37 123.12) (width 0.75) (layer "F.Cu") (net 1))
 (segment (start 179.244499 114.795501) (end 179.854098 114.795501) (width 0.15) (layer "F.Cu") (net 1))
 (segment (start 180.175948 116.400948) (end 180.275 116.5) (width 0.75) (layer "F.Cu") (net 1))
 (via (at 183 124.75) (size 1.5) (drill 1) (layers "F.Cu" "B.Cu") (free yes) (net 1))
 (segment (start 175.923595 122.343595) (end 175.9 122.32) (width 0.25) (layer "F.Cu") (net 9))
 (segment (start 177.53957 122.343595) (end 175.923595 122.343595) (width 0.25) (layer "F.Cu") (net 9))
 (segment (start 175.9 119.32) (end 177.21 119.32) (width 0.25) (layer "F.Cu") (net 5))
 (segment (start 177.21 119.32) (end 177.49 119.6) (width 0.25) (layer "F.Cu") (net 5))
 (segment (start 175.922949 119.342949) (end 175.9 119.32) (width 0.25) (layer "F.Cu") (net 5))
 (segment (start 187 118.75) (end 187 117.49) (width 0.75) (layer "F.Cu") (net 25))
 (segment (start 187 118.75) (end 187 123.75) (width 0.75) (layer "F.Cu") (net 25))
 (segment (start 187 117.49) (end 186.51 117) (width 0.75) (layer "F.Cu") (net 25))
 (segment (start 187 123.75) (end 188 124.75) (width 0.75) (layer "F.Cu") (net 25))
 (via (at 188 124.75) (size 1.5) (drill 1) (layers "F.Cu" "B.Cu") (free yes) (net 25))
 (via (at 187.8 112.05) (size 0.8) (drill 0.5) (layers "F.Cu" "B.Cu") (free yes) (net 25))
 (segment (start 184.47 120.27) (end 184.47 117.095) (width 0.75) (layer "F.Cu") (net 2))
 (segment (start 184.375 117) (end 184 116.625) (width 0.75) (layer "F.Cu") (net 2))
 (segment (start 184.47 117.095) (end 184.375 117) (width 0.75) (layer "F.Cu") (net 2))
 (segment (start 185.56 117) (end 184.375 117) (width 0.75) (layer "F.Cu") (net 2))
 (segment (start 191.32 113.55) (end 191.35 113.58) (width 0.2) (layer "F.Cu") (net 44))
 (segment (start 191.35 113.58) (end 191.35 114.75) (width 0.2) (layer "F.Cu") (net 44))
 (segment (start 189.4 112.15) (end 189.3 112.05) (width 0.2) (layer "F.Cu") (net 50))
 (via (at 189.3 112.05) (size 0.8) (drill 0.5) (layers "F.Cu" "B.Cu") (free yes) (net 50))
 (segment (start 190.25 116.65) (end 189.265 116.65) (width 0.2) (layer "F.Cu") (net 14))
 (segment (start 189.265 116.65) (end 189.165 116.55) (width 0.2) (layer "F.Cu") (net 14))
 (segment (start 190.25 116.25) (end 189.75 116.25) (width 0.2) (layer "F.Cu") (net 3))
 (segment (start 180.134612 113.201869) (end 180.134612 114.104221) (width 0.25) (layer "F.Cu") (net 3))
 (segment (start 189.75 116.25) (end 189.55 116.05) (width 0.2) (layer "F.Cu") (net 3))
 (segment (start 190.25 116.25) (end 191.75 116.25) (width 0.2) (layer "F.Cu") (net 3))
 (segment (start 178.444499 112.935501) (end 178.444499 113.865501) (width 0.2) (layer "F.Cu") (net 3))
 (segment (start 179.309154 113.865501) (end 179.553771 114.110118) (width 0.25) (layer "F.Cu") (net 3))
 (segment (start 180.134612 114.104221) (end 180.128715 114.110118) (width 0.25) (layer "F.Cu") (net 3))
 (segment (start 176.742877 114.122671) (end 178.187329 114.122671) (width 0.25) (layer "F.Cu") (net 3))
 (segment (start 188.825001 116.05) (end 188.525 116.350001) (width 0.2) (layer "F.Cu") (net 3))
 (segment (start 179.553771 114.110118) (end 180.128715 114.110118) (width 0.25) (layer "F.Cu") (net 3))
 (segment (start 178.444499 113.865501) (end 179.309154 113.865501) (width 0.25) (layer "F.Cu") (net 3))
 (segment (start 178.187329 114.122671) (end 178.444499 113.865501) (width 0.25) (layer "F.Cu") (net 3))
 (segment (start 189.55 116.05) (end 188.825001 116.05) (width 0.2) (layer "F.Cu") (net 3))
 (via (at 188.525 116.55) (size 0.4) (drill 0.2) (layers "F.Cu" "B.Cu") (free yes) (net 3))
 (via (at 191.75 116.25) (size 0.8) (drill 0.4) (layers "F.Cu" "B.Cu") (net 3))
 (via (at 190.5 124.75) (size 1.5) (drill 1) (layers "F.Cu" "B.Cu") (free yes) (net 3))
 (via (at 186.3 112.05) (size 0.8) (drill 0.5) (layers "F.Cu" "B.Cu") (free yes) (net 3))
 (via (at 179.7 124.25) (size 0.8) (drill 0.4) (layers "F.Cu" "B.Cu") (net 3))
 (via (at 185.5 124.75) (size 1.5) (drill 1) (layers "F.Cu" "B.Cu") (free yes) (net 3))
 (segment (start 191.7 116.25) (end 191.75 116.25) (width 0.2) (layer "B.Cu") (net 3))
 (segment (start 191.19 121.51) (end 191.7 121) (width 0.25) (layer "F.Cu") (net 11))
 (segment (start 190 121.51) (end 191.19 121.51) (width 0.25) (layer "F.Cu") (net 11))
 (segment (start 191.7 122.8) (end 190.5 122.8) (width 0.25) (layer "F.Cu") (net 23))
 (segment (start 190.45 122.75) (end 190.5 122.8) (width 0.25) (layer "F.Cu") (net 23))
 (segment (start 190.01 122.75) (end 190.45 122.75) (width 0.25) (layer "F.Cu") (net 23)))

